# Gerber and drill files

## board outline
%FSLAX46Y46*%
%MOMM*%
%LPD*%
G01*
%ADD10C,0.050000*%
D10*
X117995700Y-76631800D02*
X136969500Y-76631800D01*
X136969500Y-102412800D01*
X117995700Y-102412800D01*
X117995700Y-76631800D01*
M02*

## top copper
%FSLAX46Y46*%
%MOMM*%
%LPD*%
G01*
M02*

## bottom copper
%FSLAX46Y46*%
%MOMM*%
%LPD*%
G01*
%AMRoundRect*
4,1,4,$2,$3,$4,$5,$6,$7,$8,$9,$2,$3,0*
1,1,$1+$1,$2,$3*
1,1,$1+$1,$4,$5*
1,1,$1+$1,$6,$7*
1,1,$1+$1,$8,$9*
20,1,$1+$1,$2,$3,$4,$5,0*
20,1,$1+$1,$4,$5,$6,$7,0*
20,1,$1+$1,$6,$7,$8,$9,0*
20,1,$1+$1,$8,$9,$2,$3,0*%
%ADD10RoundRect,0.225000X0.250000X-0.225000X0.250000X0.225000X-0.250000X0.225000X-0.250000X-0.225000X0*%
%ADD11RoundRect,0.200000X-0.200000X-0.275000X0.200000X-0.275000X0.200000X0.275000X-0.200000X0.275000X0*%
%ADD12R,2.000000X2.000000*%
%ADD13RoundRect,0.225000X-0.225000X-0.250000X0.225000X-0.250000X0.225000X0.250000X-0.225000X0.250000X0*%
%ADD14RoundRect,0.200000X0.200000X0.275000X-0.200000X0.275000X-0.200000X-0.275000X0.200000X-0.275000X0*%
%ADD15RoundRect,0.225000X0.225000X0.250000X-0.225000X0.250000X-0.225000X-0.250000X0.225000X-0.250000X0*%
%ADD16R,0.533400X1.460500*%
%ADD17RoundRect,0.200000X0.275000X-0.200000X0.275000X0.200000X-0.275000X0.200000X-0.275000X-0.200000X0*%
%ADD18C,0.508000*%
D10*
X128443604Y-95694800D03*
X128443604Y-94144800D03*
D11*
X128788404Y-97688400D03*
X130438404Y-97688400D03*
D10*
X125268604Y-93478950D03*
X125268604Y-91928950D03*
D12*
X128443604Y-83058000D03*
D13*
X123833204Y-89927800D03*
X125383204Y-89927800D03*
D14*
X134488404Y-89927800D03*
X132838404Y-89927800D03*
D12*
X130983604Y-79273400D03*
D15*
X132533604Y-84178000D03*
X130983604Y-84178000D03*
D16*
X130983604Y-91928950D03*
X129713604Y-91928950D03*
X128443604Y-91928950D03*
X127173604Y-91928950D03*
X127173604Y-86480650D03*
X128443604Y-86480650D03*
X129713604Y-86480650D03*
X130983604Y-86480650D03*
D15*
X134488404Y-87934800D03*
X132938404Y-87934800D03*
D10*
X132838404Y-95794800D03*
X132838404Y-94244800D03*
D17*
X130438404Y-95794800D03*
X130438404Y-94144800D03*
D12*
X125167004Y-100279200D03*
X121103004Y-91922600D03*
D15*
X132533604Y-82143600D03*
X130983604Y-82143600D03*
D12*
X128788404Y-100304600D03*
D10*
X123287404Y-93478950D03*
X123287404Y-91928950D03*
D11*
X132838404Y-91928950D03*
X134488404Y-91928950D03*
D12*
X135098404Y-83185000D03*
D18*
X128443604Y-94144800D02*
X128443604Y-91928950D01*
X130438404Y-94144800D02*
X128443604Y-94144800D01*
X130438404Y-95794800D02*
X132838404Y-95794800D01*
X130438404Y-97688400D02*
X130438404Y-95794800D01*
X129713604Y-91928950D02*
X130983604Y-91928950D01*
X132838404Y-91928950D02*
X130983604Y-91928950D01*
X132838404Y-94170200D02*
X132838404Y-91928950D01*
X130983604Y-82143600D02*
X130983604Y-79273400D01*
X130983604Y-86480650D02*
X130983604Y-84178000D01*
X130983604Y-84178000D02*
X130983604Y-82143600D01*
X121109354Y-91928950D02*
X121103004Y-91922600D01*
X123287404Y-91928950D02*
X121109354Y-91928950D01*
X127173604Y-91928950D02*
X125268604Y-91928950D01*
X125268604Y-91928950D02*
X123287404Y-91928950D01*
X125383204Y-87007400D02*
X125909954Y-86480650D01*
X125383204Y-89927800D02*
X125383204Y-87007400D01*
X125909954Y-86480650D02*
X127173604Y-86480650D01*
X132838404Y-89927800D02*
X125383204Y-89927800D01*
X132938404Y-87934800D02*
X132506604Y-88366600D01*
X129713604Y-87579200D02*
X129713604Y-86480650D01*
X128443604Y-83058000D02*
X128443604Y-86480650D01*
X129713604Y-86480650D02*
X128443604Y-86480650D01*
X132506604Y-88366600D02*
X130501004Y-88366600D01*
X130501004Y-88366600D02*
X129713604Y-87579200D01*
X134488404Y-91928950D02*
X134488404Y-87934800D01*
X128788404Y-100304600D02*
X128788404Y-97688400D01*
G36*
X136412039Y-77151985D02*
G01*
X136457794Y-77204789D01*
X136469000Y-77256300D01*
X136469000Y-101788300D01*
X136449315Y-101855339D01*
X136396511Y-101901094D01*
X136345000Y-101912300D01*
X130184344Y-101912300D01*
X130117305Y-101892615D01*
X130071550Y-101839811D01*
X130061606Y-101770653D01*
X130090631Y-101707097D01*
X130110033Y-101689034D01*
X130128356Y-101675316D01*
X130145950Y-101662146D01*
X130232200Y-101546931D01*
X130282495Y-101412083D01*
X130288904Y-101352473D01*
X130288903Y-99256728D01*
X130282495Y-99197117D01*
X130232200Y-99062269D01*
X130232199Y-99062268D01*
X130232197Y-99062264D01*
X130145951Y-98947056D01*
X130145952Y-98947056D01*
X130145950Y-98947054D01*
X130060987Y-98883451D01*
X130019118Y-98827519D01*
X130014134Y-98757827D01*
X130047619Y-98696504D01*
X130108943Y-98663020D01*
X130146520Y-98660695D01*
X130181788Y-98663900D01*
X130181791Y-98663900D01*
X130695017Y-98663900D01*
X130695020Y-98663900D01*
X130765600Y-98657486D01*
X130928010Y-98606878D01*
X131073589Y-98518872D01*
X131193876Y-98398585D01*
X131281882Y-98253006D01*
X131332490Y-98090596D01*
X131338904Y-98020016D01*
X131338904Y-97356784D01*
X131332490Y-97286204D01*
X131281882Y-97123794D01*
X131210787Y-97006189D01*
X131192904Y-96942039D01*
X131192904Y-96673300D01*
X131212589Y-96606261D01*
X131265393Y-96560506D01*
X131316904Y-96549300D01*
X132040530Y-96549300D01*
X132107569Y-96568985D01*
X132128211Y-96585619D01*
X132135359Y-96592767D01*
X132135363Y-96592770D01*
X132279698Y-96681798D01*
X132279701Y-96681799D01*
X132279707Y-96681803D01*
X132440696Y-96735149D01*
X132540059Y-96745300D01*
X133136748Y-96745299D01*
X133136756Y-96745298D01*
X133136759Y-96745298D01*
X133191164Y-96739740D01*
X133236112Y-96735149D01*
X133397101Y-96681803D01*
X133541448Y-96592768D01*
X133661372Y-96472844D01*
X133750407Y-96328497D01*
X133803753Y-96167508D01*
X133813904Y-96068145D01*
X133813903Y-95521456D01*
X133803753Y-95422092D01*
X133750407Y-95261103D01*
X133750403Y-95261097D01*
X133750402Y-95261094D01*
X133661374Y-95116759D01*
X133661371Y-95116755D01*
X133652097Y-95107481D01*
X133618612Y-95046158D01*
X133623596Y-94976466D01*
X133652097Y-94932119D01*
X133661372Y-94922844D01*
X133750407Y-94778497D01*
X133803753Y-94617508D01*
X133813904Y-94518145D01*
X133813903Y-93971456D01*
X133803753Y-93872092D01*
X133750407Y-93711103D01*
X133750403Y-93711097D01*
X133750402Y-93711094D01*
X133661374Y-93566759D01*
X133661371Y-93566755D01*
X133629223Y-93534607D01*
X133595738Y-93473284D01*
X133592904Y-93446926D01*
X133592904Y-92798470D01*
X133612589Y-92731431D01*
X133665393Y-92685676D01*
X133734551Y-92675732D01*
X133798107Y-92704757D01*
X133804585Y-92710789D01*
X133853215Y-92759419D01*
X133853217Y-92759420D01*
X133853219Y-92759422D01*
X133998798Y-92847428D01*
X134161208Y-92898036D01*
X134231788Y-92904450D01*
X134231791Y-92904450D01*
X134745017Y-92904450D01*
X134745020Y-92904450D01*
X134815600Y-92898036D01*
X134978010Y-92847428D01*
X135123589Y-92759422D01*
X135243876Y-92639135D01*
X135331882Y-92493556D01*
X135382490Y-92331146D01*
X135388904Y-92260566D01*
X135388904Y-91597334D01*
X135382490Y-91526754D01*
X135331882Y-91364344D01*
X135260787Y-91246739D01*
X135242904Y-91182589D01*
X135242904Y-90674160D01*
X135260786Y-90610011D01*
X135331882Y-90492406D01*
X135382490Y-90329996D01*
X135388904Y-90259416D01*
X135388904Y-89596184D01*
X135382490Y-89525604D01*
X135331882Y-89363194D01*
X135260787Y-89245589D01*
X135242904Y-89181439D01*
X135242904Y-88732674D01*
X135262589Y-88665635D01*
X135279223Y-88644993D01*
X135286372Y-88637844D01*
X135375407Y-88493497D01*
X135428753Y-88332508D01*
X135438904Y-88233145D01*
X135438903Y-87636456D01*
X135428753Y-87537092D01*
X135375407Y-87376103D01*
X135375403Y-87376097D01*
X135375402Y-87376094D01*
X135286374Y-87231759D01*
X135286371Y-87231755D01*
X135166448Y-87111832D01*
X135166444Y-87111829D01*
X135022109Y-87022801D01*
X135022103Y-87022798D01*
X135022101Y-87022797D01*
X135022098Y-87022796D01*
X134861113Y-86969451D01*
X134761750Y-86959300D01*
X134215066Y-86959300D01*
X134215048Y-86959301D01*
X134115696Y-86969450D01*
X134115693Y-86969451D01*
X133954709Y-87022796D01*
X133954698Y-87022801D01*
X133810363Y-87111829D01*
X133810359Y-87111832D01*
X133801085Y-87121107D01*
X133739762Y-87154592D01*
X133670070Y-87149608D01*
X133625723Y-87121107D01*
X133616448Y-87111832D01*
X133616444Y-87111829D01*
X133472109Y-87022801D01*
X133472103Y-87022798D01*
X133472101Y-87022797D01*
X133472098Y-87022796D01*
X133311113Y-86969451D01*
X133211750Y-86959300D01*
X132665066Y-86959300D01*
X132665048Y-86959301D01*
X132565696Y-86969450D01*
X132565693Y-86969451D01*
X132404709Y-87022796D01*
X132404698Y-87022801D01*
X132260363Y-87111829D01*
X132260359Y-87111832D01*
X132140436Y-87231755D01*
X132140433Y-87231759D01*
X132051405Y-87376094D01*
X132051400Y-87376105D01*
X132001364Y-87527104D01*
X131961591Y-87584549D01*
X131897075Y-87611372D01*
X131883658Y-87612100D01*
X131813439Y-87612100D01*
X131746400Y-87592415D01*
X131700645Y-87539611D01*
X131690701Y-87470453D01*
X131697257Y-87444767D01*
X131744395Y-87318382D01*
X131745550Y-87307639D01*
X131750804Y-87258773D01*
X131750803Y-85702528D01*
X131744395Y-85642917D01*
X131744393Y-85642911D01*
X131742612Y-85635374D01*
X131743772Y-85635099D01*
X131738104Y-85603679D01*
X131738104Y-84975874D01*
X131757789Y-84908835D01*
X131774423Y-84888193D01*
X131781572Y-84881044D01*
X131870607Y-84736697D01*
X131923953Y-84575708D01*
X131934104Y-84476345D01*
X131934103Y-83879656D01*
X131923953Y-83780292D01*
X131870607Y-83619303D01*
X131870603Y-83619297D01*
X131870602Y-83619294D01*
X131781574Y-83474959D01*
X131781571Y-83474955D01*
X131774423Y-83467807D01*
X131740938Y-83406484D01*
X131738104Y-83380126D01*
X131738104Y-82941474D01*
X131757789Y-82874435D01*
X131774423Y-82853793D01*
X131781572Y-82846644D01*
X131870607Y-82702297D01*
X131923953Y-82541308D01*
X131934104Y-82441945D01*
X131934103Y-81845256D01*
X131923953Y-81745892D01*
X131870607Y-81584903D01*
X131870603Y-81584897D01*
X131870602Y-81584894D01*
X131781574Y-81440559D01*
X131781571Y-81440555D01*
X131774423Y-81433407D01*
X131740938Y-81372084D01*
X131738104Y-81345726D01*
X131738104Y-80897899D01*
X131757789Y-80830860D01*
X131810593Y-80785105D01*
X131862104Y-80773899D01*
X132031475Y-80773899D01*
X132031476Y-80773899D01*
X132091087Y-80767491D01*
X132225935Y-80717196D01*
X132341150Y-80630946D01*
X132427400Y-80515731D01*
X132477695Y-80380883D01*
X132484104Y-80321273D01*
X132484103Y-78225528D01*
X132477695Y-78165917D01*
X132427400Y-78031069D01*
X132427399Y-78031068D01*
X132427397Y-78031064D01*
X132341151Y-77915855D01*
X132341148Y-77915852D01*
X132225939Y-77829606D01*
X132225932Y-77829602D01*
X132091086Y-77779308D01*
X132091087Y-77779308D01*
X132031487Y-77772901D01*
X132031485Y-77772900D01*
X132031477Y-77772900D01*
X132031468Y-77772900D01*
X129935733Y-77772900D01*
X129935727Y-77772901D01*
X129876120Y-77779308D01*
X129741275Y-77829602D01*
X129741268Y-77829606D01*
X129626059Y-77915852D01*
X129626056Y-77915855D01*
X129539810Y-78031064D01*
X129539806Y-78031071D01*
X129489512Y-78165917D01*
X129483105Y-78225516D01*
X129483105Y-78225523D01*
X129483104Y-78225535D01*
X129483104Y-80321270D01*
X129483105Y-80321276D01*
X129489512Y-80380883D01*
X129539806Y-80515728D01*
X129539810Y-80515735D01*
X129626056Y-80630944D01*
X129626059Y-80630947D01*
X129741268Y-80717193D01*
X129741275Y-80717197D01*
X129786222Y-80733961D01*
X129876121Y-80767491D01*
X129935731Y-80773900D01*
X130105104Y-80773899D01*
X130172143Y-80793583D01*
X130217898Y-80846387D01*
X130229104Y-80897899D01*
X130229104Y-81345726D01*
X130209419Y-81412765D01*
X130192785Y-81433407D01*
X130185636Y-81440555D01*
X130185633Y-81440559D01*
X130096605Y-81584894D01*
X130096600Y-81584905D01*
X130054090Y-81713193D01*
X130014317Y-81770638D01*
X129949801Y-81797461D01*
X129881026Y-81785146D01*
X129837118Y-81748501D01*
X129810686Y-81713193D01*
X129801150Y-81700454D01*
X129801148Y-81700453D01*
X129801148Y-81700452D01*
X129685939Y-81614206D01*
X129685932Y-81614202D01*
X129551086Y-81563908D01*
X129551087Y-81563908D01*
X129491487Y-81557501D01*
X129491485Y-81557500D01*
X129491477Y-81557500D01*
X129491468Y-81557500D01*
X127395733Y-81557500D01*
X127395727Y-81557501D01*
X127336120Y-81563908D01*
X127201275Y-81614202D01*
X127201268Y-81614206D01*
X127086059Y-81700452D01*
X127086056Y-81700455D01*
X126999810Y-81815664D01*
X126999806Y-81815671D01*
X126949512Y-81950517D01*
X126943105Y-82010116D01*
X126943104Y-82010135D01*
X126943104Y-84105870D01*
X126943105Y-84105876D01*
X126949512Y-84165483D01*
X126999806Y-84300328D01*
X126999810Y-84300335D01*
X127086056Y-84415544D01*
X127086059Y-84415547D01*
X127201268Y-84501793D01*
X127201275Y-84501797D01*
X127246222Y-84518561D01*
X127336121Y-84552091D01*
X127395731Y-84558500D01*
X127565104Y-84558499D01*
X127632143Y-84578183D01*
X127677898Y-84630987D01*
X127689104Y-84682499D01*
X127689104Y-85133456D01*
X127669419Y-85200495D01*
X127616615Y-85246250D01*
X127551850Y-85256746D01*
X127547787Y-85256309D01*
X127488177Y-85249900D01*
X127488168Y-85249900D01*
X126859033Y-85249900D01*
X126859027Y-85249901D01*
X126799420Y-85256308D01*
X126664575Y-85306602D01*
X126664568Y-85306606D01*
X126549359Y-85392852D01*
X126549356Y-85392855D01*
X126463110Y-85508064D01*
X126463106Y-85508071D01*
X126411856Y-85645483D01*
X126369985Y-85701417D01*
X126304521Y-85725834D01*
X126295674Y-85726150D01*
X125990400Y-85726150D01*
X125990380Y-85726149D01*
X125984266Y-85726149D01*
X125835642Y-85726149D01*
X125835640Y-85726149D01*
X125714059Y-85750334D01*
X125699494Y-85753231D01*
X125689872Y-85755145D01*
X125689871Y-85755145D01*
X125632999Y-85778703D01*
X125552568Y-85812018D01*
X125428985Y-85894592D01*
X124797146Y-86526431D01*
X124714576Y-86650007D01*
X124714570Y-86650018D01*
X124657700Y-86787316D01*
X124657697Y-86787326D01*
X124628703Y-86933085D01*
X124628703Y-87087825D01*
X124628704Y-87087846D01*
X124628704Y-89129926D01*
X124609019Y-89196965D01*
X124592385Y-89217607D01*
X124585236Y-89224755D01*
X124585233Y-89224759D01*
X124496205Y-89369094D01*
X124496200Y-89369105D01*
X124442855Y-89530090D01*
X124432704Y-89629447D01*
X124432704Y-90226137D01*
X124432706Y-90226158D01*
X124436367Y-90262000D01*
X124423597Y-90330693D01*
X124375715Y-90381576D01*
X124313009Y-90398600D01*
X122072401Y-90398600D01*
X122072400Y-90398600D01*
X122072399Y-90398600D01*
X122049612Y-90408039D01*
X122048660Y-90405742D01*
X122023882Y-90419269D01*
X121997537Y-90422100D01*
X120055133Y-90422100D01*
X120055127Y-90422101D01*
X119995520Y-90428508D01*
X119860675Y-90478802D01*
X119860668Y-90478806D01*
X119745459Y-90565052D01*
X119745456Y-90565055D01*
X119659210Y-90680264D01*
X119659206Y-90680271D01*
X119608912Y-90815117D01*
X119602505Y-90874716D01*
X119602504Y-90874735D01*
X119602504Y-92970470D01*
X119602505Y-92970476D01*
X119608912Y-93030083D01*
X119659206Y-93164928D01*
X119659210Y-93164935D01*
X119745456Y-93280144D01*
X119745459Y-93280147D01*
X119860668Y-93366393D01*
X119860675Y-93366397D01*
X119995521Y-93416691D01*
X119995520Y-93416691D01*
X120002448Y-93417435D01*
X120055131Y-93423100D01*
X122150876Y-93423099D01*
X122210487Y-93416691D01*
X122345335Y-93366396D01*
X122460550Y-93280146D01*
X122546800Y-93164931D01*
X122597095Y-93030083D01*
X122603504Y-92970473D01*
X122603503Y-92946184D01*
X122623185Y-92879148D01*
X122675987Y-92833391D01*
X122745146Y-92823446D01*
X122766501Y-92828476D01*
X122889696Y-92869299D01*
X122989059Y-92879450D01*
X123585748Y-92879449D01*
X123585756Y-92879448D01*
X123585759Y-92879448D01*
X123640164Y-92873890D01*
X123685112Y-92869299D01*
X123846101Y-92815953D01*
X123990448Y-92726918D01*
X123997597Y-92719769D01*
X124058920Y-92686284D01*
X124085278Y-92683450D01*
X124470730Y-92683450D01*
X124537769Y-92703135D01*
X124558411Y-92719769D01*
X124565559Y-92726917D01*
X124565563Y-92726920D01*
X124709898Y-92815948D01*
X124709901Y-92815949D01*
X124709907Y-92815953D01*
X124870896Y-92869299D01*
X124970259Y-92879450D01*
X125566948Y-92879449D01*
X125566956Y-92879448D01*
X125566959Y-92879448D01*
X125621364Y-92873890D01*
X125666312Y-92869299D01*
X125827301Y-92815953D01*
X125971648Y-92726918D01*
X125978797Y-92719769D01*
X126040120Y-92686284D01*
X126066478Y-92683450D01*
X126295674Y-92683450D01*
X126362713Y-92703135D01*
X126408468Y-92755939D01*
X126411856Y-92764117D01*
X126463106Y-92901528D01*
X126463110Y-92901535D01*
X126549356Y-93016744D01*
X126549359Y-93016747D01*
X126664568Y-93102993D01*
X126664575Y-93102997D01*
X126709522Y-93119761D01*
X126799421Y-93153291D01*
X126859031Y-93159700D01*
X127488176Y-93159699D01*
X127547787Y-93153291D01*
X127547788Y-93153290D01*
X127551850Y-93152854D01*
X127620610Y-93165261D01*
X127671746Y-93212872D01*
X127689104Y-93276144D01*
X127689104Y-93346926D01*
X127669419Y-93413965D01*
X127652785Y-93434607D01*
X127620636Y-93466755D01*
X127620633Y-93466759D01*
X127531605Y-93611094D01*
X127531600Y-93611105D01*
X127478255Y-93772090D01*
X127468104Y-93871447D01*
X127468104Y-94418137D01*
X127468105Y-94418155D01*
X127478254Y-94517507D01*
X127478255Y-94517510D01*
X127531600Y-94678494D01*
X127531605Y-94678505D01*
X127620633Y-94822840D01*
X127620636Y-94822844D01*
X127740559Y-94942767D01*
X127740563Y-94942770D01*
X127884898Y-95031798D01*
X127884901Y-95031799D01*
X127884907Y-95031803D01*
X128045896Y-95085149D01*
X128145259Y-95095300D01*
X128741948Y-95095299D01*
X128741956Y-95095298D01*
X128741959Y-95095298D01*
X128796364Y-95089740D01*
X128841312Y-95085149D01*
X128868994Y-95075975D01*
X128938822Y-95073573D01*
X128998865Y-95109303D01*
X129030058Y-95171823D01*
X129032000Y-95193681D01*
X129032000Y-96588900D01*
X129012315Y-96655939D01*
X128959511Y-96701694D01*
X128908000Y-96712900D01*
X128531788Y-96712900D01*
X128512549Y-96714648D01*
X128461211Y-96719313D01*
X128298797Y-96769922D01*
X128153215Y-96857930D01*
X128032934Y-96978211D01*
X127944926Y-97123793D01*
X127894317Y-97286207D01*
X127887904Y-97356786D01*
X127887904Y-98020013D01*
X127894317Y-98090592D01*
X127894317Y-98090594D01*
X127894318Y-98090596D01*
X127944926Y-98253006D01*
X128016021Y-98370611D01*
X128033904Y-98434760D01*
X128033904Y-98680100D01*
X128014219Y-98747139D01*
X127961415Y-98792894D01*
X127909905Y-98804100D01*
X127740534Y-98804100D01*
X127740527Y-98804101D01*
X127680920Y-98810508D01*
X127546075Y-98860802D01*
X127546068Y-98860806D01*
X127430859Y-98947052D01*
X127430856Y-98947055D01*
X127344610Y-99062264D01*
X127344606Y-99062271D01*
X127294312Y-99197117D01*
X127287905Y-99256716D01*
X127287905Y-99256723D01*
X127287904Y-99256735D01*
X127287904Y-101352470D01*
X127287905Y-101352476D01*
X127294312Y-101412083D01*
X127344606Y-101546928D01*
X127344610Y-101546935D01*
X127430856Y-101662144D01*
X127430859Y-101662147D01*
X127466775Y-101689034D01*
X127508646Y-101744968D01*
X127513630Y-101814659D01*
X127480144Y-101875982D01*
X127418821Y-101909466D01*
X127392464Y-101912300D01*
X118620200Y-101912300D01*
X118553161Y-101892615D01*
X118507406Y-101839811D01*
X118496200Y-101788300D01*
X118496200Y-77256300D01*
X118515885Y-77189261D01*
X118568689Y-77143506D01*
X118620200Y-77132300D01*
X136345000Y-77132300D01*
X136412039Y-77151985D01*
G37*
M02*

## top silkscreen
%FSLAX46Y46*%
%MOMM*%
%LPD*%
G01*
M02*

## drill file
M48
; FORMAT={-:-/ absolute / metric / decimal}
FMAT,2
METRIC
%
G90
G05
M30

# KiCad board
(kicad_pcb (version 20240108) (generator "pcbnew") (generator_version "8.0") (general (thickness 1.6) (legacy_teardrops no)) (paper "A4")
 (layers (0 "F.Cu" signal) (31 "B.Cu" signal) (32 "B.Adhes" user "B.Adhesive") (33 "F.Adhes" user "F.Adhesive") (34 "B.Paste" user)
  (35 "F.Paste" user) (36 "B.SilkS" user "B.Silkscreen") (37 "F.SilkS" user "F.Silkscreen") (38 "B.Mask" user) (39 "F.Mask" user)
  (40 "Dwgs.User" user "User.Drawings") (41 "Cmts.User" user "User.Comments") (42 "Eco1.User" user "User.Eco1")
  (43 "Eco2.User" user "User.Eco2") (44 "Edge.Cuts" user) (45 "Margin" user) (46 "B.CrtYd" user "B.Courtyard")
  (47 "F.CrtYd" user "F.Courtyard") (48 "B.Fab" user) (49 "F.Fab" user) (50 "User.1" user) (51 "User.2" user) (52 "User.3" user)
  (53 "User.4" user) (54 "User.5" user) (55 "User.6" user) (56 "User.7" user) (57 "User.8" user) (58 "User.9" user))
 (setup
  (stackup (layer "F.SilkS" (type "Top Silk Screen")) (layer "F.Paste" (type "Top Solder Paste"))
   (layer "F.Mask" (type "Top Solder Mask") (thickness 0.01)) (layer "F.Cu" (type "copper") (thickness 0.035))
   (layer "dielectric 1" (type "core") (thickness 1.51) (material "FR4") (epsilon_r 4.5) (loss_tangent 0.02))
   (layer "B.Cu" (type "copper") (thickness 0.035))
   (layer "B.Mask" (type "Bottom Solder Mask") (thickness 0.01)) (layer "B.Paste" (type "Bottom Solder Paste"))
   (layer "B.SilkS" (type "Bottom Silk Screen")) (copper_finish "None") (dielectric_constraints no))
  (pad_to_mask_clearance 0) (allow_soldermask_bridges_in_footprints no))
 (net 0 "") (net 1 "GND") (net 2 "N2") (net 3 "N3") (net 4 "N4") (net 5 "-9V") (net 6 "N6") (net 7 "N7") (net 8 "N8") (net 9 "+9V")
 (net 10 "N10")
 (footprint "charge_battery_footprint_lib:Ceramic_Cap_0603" (layer "B.Cu") (at 128.443604 94.9198 90)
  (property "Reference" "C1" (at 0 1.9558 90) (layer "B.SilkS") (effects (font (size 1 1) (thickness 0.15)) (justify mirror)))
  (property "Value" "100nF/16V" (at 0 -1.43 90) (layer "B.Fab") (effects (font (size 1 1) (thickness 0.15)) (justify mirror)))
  (pad "1" smd roundrect (at -0.775 0 90) (size 0.9 0.95) (layers "B.Cu" "B.Paste" "B.Mask") (roundrect_rratio 0.25) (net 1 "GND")
   (solder_mask_margin 0.102))
  (pad "2" smd roundrect (at 0.775 0 90) (size 0.9 0.95) (layers "B.Cu" "B.Paste" "B.Mask") (roundrect_rratio 0.25) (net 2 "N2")
   (solder_mask_margin 0.102)))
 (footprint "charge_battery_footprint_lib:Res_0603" (layer "B.Cu") (at 128.254604 97.0788)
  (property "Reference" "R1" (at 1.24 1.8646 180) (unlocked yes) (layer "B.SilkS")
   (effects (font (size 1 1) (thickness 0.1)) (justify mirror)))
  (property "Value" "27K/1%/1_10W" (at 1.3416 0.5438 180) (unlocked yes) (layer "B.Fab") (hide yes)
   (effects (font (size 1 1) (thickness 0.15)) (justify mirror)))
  (pad "1" smd roundrect (at 0.5338 0.6096) (size 0.8 0.95) (layers "B.Cu" "B.Paste" "B.Mask") (roundrect_rratio 0.25) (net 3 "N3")
   (solder_mask_margin 0.102) (solder_paste_margin_ratio -0.01))
  (pad "2" smd roundrect (at 2.1838 0.6096) (size 0.8 0.95) (layers "B.Cu" "B.Paste" "B.Mask") (roundrect_rratio 0.25) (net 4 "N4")
   (solder_mask_margin 0.102)))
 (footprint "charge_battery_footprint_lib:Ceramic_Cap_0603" (layer "B.Cu") (at 125.268604 92.70395 90)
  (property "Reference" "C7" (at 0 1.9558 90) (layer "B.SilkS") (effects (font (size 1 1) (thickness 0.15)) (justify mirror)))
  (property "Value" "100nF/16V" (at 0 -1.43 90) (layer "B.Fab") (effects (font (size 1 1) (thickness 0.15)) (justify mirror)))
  (pad "1" smd roundrect (at -0.775 0 90) (size 0.9 0.95) (layers "B.Cu" "B.Paste" "B.Mask") (roundrect_rratio 0.25) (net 1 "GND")
   (solder_mask_margin 0.102))
  (pad "2" smd roundrect (at 0.775 0 90) (size 0.9 0.95) (layers "B.Cu" "B.Paste" "B.Mask") (roundrect_rratio 0.25) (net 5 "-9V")
   (solder_mask_margin 0.102)))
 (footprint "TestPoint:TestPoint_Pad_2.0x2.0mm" (layer "B.Cu") (at 128.443604 83.058 180)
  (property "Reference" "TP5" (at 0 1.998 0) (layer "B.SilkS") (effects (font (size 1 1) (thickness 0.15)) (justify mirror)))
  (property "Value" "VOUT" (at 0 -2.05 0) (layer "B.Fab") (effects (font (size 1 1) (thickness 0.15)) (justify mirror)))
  (pad "1" smd rect (at 0 0 180) (size 2 2) (layers "B.Cu" "B.Mask") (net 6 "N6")))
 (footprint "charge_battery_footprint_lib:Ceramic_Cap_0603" (layer "B.Cu") (at 124.608204 89.9278)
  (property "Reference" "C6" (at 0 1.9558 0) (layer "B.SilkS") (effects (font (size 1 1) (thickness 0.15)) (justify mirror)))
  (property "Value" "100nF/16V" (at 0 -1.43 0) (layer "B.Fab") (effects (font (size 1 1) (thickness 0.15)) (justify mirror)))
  (pad "1" smd roundrect (at -0.775 0) (size 0.9 0.95) (layers "B.Cu" "B.Paste" "B.Mask") (roundrect_rratio 0.25) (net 1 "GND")
   (solder_mask_margin 0.102))
  (pad "2" smd roundrect (at 0.775 0) (size 0.9 0.95) (layers "B.Cu" "B.Paste" "B.Mask") (roundrect_rratio 0.25) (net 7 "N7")
   (solder_mask_margin 0.102)))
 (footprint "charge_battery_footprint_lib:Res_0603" (layer "B.Cu") (at 135.022204 90.5374 180)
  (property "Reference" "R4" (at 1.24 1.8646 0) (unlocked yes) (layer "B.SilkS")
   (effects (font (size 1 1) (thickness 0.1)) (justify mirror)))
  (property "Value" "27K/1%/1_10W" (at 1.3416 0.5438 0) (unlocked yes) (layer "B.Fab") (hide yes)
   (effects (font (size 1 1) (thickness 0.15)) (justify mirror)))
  (pad "1" smd roundrect (at 0.5338 0.6096 180) (size 0.8 0.95) (layers "B.Cu" "B.Paste" "B.Mask") (roundrect_rratio 0.25) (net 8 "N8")
   (solder_mask_margin 0.102) (solder_paste_margin_ratio -0.01))
  (pad "2" smd roundrect (at 2.1838 0.6096 180) (size 0.8 0.95) (layers "B.Cu" "B.Paste" "B.Mask") (roundrect_rratio 0.25) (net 7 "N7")
   (solder_mask_margin 0.102)))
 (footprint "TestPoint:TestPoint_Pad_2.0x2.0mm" (layer "B.Cu") (at 130.983604 79.2734 180)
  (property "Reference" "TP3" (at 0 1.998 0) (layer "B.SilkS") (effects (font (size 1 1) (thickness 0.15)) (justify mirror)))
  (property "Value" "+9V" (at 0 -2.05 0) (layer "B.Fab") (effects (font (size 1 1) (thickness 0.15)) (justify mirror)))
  (pad "1" smd rect (at 0 0 180) (size 2 2) (layers "B.Cu" "B.Mask") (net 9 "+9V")))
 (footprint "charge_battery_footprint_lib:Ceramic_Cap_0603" (layer "B.Cu") (at 131.758604 84.178 180)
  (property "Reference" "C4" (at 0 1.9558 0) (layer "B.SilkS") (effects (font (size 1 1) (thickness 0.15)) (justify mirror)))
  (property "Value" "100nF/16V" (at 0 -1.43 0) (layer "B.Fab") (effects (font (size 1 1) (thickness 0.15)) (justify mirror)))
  (pad "1" smd roundrect (at -0.775 0 180) (size 0.9 0.95) (layers "B.Cu" "B.Paste" "B.Mask") (roundrect_rratio 0.25) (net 1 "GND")
   (solder_mask_margin 0.102))
  (pad "2" smd roundrect (at 0.775 0 180) (size 0.9 0.95) (layers "B.Cu" "B.Paste" "B.Mask") (roundrect_rratio 0.25) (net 9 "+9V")
   (solder_mask_margin 0.102)))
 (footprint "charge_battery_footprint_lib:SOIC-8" (layer "B.Cu") (at 129.078604 89.2048 90)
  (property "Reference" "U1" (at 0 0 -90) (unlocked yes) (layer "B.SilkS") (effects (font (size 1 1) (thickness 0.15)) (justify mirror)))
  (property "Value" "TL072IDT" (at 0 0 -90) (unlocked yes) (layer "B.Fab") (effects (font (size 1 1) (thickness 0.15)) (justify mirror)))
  (pad "1" smd rect (at -2.72415 1.905 90) (size 1.4605 0.5334) (layers "B.Cu" "B.Paste" "B.Mask") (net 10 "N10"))
  (pad "2" smd rect (at -2.72415 0.635 90) (size 1.4605 0.5334) (layers "B.Cu" "B.Paste" "B.Mask") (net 10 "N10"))
  (pad "3" smd rect (at -2.72415 -0.635 90) (size 1.4605 0.5334) (layers "B.Cu" "B.Paste" "B.Mask") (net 2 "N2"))
  (pad "4" smd rect (at -2.72415 -1.905 90) (size 1.4605 0.5334) (layers "B.Cu" "B.Paste" "B.Mask") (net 5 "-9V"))
  (pad "5" smd rect (at 2.72415 -1.905 90) (size 1.4605 0.5334) (layers "B.Cu" "B.Paste" "B.Mask") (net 7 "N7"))
  (pad "6" smd rect (at 2.72415 -0.635 90) (size 1.4605 0.5334) (layers "B.Cu" "B.Paste" "B.Mask") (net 6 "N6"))
  (pad "7" smd rect (at 2.72415 0.635 90) (size 1.4605 0.5334) (layers "B.Cu" "B.Paste" "B.Mask") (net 6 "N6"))
  (pad "8" smd rect (at 2.72415 1.905 90) (size 1.4605 0.5334) (layers "B.Cu" "B.Paste" "B.Mask") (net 9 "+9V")))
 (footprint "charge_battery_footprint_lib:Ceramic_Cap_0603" (layer "B.Cu") (at 133.713404 87.9348 180)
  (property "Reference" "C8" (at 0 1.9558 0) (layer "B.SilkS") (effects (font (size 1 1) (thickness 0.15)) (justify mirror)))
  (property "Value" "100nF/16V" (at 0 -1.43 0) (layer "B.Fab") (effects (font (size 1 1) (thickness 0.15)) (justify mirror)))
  (pad "1" smd roundrect (at -0.775 0 180) (size 0.9 0.95) (layers "B.Cu" "B.Paste" "B.Mask") (roundrect_rratio 0.25) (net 8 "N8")
   (solder_mask_margin 0.102))
  (pad "2" smd roundrect (at 0.775 0 180) (size 0.9 0.95) (layers "B.Cu" "B.Paste" "B.Mask") (roundrect_rratio 0.25) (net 6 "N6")
   (solder_mask_margin 0.102)))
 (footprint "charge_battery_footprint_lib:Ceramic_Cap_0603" (layer "B.Cu") (at 132.838404 95.0198 90)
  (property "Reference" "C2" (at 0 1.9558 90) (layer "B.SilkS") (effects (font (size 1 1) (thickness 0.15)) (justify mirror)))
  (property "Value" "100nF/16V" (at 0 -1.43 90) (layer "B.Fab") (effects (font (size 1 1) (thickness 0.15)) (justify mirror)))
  (pad "1" smd roundrect (at -0.775 0 90) (size 0.9 0.95) (layers "B.Cu" "B.Paste" "B.Mask") (roundrect_rratio 0.25) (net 4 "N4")
   (solder_mask_margin 0.102))
  (pad "2" smd roundrect (at 0.775 0 90) (size 0.9 0.95) (layers "B.Cu" "B.Paste" "B.Mask") (roundrect_rratio 0.25) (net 10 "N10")
   (solder_mask_margin 0.102)))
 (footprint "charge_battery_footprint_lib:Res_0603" (layer "B.Cu") (at 129.828804 96.3286 90)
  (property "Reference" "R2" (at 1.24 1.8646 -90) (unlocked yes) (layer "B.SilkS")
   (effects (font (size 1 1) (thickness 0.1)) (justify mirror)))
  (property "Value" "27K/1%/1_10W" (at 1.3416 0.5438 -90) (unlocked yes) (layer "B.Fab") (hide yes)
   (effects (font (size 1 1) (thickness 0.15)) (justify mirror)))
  (pad "1" smd roundrect (at 0.5338 0.6096 90) (size 0.8 0.95) (layers "B.Cu" "B.Paste" "B.Mask") (roundrect_rratio 0.25) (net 4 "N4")
   (solder_mask_margin 0.102) (solder_paste_margin_ratio -0.01))
  (pad "2" smd roundrect (at 2.1838 0.6096 90) (size 0.8 0.95) (layers "B.Cu" "B.Paste" "B.Mask") (roundrect_rratio 0.25) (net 2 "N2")
   (solder_mask_margin 0.102)))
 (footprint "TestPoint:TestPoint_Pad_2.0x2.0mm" (layer "B.Cu") (at 125.167004 100.2792 180)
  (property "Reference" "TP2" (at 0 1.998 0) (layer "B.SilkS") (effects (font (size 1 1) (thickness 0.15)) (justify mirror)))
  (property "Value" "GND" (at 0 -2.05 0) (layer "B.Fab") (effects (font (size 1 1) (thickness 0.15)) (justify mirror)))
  (pad "1" smd rect (at 0 0 180) (size 2 2) (layers "B.Cu" "B.Mask") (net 1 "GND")))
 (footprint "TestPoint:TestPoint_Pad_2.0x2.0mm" (layer "B.Cu") (at 121.103004 91.9226 180)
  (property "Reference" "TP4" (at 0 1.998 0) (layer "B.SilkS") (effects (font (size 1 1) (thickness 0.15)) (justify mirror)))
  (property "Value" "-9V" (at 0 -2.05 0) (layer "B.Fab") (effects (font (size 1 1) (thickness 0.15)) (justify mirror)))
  (pad "1" smd rect (at 0 0 180) (size 2 2) (layers "B.Cu" "B.Mask") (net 5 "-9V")))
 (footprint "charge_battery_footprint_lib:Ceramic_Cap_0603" (layer "B.Cu") (at 131.758604 82.1436 180)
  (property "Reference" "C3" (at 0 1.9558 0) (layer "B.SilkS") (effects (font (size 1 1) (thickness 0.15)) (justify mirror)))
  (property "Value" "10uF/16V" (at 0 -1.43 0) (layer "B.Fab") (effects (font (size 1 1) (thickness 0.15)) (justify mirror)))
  (pad "1" smd roundrect (at -0.775 0 180) (size 0.9 0.95) (layers "B.Cu" "B.Paste" "B.Mask") (roundrect_rratio 0.25) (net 1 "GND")
   (solder_mask_margin 0.102))
  (pad "2" smd roundrect (at 0.775 0 180) (size 0.9 0.95) (layers "B.Cu" "B.Paste" "B.Mask") (roundrect_rratio 0.25) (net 9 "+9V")
   (solder_mask_margin 0.102)))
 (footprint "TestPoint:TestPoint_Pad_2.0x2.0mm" (layer "B.Cu") (at 128.788404 100.3046 180)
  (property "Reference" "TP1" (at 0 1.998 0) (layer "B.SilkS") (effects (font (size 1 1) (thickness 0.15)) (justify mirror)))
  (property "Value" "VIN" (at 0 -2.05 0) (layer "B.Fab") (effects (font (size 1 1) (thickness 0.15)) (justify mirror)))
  (pad "1" smd rect (at 0 0 180) (size 2 2) (layers "B.Cu" "B.Mask") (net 3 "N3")))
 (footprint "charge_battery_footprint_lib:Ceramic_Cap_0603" (layer "B.Cu") (at 123.287404 92.70395 90)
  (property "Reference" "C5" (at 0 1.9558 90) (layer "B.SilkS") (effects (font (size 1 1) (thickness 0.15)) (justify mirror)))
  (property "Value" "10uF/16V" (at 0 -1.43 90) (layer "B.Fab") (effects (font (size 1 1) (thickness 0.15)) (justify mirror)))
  (pad "1" smd roundrect (at -0.775 0 90) (size 0.9 0.95) (layers "B.Cu" "B.Paste" "B.Mask") (roundrect_rratio 0.25) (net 1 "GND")
   (solder_mask_margin 0.102))
  (pad "2" smd roundrect (at 0.775 0 90) (size 0.9 0.95) (layers "B.Cu" "B.Paste" "B.Mask") (roundrect_rratio 0.25) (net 5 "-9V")
   (solder_mask_margin 0.102)))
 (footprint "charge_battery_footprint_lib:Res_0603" (layer "B.Cu") (at 132.304604 91.31935)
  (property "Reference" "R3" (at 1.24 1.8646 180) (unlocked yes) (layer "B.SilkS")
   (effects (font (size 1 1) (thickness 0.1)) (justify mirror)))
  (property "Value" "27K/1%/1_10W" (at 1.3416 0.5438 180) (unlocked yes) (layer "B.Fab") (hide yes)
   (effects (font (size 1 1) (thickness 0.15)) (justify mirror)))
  (pad "1" smd roundrect (at 0.5338 0.6096) (size 0.8 0.95) (layers "B.Cu" "B.Paste" "B.Mask") (roundrect_rratio 0.25) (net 10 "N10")
   (solder_mask_margin 0.102) (solder_paste_margin_ratio -0.01))
  (pad "2" smd roundrect (at 2.1838 0.6096) (size 0.8 0.95) (layers "B.Cu" "B.Paste" "B.Mask") (roundrect_rratio 0.25) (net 8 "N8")
   (solder_mask_margin 0.102)))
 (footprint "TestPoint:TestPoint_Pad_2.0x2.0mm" (layer "B.Cu") (at 135.098404 83.185 180)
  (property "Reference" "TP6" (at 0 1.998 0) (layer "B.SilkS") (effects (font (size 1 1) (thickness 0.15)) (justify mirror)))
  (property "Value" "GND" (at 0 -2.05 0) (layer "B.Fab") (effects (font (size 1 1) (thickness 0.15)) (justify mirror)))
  (pad "1" smd rect (at 0 0 180) (size 2 2) (layers "B.Cu" "B.Mask") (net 1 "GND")))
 (gr_rect (start 117.9957 76.6318) (end 136.9695 102.4128) (stroke (width 0.05) (type default)) (fill none) (layer "Edge.Cuts"))
 (segment (start 128.443604 94.1448) (end 128.443604 91.92895) (width 0.508) (layer "B.Cu") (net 2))
 (segment (start 130.438404 94.1448) (end 128.443604 94.1448) (width 0.508) (layer "B.Cu") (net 2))
 (segment (start 130.438404 95.7948) (end 132.838404 95.7948) (width 0.508) (layer "B.Cu") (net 4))
 (segment (start 130.438404 97.6884) (end 130.438404 95.7948) (width 0.508) (layer "B.Cu") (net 4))
 (segment (start 129.713604 91.92895) (end 130.983604 91.92895) (width 0.508) (layer "B.Cu") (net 10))
 (segment (start 132.838404 91.92895) (end 130.983604 91.92895) (width 0.508) (layer "B.Cu") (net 10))
 (segment (start 132.838404 94.1702) (end 132.838404 91.92895) (width 0.508) (layer "B.Cu") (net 10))
 (segment (start 130.983604 82.1436) (end 130.983604 79.2734) (width 0.508) (layer "B.Cu") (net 9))
 (segment (start 130.983604 86.48065) (end 130.983604 84.178) (width 0.508) (layer "B.Cu") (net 9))
 (segment (start 130.983604 84.178) (end 130.983604 82.1436) (width 0.508) (layer "B.Cu") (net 9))
 (segment (start 121.109354 91.92895) (end 121.103004 91.9226) (width 0.508) (layer "B.Cu") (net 5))
 (segment (start 123.287404 91.92895) (end 121.109354 91.92895) (width 0.508) (layer "B.Cu") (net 5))
 (segment (start 127.173604 91.92895) (end 125.268604 91.92895) (width 0.508) (layer "B.Cu") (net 5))
 (segment (start 125.268604 91.92895) (end 123.287404 91.92895) (width 0.508) (layer "B.Cu") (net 5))
 (segment (start 125.383204 87.0074) (end 125.909954 86.48065) (width 0.508) (layer "B.Cu") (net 7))
 (segment (start 125.383204 89.9278) (end 125.383204 87.0074) (width 0.508) (layer "B.Cu") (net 7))
 (segment (start 125.909954 86.48065) (end 127.173604 86.48065) (width 0.508) (layer "B.Cu") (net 7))
 (segment (start 132.838404 89.9278) (end 125.383204 89.9278) (width 0.508) (layer "B.Cu") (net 7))
 (segment (start 132.938404 87.9348) (end 132.506604 88.3666) (width 0.508) (layer "B.Cu") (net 6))
 (segment (start 129.713604 87.5792) (end 129.713604 86.48065) (width 0.508) (layer "B.Cu") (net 6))
 (segment (start 128.443604 83.058) (end 128.443604 86.48065) (width 0.508) (layer "B.Cu") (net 6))
 (segment (start 129.713604 86.48065) (end 128.443604 86.48065) (width 0.508) (layer "B.Cu") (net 6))
 (segment (start 132.506604 88.3666) (end 130.501004 88.3666) (width 0.508) (layer "B.Cu") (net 6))
 (segment (start 130.501004 88.3666) (end 129.713604 87.5792) (width 0.508) (layer "B.Cu") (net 6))
 (segment (start 134.488404 91.92895) (end 134.488404 87.9348) (width 0.508) (layer "B.Cu") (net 8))
 (segment (start 128.788404 100.3046) (end 128.788404 97.6884) (width 0.508) (layer "B.Cu") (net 3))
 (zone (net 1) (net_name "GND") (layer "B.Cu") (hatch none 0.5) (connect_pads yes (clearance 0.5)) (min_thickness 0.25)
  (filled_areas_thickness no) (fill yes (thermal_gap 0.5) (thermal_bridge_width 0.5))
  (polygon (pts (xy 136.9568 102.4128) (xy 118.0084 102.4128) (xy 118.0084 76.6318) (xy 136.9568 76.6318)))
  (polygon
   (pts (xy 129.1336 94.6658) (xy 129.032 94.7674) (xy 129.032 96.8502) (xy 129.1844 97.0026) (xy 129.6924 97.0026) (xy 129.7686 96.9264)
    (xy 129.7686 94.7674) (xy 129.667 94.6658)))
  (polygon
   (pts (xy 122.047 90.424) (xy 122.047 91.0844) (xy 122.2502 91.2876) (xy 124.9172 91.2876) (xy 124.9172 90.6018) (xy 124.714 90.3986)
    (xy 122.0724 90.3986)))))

